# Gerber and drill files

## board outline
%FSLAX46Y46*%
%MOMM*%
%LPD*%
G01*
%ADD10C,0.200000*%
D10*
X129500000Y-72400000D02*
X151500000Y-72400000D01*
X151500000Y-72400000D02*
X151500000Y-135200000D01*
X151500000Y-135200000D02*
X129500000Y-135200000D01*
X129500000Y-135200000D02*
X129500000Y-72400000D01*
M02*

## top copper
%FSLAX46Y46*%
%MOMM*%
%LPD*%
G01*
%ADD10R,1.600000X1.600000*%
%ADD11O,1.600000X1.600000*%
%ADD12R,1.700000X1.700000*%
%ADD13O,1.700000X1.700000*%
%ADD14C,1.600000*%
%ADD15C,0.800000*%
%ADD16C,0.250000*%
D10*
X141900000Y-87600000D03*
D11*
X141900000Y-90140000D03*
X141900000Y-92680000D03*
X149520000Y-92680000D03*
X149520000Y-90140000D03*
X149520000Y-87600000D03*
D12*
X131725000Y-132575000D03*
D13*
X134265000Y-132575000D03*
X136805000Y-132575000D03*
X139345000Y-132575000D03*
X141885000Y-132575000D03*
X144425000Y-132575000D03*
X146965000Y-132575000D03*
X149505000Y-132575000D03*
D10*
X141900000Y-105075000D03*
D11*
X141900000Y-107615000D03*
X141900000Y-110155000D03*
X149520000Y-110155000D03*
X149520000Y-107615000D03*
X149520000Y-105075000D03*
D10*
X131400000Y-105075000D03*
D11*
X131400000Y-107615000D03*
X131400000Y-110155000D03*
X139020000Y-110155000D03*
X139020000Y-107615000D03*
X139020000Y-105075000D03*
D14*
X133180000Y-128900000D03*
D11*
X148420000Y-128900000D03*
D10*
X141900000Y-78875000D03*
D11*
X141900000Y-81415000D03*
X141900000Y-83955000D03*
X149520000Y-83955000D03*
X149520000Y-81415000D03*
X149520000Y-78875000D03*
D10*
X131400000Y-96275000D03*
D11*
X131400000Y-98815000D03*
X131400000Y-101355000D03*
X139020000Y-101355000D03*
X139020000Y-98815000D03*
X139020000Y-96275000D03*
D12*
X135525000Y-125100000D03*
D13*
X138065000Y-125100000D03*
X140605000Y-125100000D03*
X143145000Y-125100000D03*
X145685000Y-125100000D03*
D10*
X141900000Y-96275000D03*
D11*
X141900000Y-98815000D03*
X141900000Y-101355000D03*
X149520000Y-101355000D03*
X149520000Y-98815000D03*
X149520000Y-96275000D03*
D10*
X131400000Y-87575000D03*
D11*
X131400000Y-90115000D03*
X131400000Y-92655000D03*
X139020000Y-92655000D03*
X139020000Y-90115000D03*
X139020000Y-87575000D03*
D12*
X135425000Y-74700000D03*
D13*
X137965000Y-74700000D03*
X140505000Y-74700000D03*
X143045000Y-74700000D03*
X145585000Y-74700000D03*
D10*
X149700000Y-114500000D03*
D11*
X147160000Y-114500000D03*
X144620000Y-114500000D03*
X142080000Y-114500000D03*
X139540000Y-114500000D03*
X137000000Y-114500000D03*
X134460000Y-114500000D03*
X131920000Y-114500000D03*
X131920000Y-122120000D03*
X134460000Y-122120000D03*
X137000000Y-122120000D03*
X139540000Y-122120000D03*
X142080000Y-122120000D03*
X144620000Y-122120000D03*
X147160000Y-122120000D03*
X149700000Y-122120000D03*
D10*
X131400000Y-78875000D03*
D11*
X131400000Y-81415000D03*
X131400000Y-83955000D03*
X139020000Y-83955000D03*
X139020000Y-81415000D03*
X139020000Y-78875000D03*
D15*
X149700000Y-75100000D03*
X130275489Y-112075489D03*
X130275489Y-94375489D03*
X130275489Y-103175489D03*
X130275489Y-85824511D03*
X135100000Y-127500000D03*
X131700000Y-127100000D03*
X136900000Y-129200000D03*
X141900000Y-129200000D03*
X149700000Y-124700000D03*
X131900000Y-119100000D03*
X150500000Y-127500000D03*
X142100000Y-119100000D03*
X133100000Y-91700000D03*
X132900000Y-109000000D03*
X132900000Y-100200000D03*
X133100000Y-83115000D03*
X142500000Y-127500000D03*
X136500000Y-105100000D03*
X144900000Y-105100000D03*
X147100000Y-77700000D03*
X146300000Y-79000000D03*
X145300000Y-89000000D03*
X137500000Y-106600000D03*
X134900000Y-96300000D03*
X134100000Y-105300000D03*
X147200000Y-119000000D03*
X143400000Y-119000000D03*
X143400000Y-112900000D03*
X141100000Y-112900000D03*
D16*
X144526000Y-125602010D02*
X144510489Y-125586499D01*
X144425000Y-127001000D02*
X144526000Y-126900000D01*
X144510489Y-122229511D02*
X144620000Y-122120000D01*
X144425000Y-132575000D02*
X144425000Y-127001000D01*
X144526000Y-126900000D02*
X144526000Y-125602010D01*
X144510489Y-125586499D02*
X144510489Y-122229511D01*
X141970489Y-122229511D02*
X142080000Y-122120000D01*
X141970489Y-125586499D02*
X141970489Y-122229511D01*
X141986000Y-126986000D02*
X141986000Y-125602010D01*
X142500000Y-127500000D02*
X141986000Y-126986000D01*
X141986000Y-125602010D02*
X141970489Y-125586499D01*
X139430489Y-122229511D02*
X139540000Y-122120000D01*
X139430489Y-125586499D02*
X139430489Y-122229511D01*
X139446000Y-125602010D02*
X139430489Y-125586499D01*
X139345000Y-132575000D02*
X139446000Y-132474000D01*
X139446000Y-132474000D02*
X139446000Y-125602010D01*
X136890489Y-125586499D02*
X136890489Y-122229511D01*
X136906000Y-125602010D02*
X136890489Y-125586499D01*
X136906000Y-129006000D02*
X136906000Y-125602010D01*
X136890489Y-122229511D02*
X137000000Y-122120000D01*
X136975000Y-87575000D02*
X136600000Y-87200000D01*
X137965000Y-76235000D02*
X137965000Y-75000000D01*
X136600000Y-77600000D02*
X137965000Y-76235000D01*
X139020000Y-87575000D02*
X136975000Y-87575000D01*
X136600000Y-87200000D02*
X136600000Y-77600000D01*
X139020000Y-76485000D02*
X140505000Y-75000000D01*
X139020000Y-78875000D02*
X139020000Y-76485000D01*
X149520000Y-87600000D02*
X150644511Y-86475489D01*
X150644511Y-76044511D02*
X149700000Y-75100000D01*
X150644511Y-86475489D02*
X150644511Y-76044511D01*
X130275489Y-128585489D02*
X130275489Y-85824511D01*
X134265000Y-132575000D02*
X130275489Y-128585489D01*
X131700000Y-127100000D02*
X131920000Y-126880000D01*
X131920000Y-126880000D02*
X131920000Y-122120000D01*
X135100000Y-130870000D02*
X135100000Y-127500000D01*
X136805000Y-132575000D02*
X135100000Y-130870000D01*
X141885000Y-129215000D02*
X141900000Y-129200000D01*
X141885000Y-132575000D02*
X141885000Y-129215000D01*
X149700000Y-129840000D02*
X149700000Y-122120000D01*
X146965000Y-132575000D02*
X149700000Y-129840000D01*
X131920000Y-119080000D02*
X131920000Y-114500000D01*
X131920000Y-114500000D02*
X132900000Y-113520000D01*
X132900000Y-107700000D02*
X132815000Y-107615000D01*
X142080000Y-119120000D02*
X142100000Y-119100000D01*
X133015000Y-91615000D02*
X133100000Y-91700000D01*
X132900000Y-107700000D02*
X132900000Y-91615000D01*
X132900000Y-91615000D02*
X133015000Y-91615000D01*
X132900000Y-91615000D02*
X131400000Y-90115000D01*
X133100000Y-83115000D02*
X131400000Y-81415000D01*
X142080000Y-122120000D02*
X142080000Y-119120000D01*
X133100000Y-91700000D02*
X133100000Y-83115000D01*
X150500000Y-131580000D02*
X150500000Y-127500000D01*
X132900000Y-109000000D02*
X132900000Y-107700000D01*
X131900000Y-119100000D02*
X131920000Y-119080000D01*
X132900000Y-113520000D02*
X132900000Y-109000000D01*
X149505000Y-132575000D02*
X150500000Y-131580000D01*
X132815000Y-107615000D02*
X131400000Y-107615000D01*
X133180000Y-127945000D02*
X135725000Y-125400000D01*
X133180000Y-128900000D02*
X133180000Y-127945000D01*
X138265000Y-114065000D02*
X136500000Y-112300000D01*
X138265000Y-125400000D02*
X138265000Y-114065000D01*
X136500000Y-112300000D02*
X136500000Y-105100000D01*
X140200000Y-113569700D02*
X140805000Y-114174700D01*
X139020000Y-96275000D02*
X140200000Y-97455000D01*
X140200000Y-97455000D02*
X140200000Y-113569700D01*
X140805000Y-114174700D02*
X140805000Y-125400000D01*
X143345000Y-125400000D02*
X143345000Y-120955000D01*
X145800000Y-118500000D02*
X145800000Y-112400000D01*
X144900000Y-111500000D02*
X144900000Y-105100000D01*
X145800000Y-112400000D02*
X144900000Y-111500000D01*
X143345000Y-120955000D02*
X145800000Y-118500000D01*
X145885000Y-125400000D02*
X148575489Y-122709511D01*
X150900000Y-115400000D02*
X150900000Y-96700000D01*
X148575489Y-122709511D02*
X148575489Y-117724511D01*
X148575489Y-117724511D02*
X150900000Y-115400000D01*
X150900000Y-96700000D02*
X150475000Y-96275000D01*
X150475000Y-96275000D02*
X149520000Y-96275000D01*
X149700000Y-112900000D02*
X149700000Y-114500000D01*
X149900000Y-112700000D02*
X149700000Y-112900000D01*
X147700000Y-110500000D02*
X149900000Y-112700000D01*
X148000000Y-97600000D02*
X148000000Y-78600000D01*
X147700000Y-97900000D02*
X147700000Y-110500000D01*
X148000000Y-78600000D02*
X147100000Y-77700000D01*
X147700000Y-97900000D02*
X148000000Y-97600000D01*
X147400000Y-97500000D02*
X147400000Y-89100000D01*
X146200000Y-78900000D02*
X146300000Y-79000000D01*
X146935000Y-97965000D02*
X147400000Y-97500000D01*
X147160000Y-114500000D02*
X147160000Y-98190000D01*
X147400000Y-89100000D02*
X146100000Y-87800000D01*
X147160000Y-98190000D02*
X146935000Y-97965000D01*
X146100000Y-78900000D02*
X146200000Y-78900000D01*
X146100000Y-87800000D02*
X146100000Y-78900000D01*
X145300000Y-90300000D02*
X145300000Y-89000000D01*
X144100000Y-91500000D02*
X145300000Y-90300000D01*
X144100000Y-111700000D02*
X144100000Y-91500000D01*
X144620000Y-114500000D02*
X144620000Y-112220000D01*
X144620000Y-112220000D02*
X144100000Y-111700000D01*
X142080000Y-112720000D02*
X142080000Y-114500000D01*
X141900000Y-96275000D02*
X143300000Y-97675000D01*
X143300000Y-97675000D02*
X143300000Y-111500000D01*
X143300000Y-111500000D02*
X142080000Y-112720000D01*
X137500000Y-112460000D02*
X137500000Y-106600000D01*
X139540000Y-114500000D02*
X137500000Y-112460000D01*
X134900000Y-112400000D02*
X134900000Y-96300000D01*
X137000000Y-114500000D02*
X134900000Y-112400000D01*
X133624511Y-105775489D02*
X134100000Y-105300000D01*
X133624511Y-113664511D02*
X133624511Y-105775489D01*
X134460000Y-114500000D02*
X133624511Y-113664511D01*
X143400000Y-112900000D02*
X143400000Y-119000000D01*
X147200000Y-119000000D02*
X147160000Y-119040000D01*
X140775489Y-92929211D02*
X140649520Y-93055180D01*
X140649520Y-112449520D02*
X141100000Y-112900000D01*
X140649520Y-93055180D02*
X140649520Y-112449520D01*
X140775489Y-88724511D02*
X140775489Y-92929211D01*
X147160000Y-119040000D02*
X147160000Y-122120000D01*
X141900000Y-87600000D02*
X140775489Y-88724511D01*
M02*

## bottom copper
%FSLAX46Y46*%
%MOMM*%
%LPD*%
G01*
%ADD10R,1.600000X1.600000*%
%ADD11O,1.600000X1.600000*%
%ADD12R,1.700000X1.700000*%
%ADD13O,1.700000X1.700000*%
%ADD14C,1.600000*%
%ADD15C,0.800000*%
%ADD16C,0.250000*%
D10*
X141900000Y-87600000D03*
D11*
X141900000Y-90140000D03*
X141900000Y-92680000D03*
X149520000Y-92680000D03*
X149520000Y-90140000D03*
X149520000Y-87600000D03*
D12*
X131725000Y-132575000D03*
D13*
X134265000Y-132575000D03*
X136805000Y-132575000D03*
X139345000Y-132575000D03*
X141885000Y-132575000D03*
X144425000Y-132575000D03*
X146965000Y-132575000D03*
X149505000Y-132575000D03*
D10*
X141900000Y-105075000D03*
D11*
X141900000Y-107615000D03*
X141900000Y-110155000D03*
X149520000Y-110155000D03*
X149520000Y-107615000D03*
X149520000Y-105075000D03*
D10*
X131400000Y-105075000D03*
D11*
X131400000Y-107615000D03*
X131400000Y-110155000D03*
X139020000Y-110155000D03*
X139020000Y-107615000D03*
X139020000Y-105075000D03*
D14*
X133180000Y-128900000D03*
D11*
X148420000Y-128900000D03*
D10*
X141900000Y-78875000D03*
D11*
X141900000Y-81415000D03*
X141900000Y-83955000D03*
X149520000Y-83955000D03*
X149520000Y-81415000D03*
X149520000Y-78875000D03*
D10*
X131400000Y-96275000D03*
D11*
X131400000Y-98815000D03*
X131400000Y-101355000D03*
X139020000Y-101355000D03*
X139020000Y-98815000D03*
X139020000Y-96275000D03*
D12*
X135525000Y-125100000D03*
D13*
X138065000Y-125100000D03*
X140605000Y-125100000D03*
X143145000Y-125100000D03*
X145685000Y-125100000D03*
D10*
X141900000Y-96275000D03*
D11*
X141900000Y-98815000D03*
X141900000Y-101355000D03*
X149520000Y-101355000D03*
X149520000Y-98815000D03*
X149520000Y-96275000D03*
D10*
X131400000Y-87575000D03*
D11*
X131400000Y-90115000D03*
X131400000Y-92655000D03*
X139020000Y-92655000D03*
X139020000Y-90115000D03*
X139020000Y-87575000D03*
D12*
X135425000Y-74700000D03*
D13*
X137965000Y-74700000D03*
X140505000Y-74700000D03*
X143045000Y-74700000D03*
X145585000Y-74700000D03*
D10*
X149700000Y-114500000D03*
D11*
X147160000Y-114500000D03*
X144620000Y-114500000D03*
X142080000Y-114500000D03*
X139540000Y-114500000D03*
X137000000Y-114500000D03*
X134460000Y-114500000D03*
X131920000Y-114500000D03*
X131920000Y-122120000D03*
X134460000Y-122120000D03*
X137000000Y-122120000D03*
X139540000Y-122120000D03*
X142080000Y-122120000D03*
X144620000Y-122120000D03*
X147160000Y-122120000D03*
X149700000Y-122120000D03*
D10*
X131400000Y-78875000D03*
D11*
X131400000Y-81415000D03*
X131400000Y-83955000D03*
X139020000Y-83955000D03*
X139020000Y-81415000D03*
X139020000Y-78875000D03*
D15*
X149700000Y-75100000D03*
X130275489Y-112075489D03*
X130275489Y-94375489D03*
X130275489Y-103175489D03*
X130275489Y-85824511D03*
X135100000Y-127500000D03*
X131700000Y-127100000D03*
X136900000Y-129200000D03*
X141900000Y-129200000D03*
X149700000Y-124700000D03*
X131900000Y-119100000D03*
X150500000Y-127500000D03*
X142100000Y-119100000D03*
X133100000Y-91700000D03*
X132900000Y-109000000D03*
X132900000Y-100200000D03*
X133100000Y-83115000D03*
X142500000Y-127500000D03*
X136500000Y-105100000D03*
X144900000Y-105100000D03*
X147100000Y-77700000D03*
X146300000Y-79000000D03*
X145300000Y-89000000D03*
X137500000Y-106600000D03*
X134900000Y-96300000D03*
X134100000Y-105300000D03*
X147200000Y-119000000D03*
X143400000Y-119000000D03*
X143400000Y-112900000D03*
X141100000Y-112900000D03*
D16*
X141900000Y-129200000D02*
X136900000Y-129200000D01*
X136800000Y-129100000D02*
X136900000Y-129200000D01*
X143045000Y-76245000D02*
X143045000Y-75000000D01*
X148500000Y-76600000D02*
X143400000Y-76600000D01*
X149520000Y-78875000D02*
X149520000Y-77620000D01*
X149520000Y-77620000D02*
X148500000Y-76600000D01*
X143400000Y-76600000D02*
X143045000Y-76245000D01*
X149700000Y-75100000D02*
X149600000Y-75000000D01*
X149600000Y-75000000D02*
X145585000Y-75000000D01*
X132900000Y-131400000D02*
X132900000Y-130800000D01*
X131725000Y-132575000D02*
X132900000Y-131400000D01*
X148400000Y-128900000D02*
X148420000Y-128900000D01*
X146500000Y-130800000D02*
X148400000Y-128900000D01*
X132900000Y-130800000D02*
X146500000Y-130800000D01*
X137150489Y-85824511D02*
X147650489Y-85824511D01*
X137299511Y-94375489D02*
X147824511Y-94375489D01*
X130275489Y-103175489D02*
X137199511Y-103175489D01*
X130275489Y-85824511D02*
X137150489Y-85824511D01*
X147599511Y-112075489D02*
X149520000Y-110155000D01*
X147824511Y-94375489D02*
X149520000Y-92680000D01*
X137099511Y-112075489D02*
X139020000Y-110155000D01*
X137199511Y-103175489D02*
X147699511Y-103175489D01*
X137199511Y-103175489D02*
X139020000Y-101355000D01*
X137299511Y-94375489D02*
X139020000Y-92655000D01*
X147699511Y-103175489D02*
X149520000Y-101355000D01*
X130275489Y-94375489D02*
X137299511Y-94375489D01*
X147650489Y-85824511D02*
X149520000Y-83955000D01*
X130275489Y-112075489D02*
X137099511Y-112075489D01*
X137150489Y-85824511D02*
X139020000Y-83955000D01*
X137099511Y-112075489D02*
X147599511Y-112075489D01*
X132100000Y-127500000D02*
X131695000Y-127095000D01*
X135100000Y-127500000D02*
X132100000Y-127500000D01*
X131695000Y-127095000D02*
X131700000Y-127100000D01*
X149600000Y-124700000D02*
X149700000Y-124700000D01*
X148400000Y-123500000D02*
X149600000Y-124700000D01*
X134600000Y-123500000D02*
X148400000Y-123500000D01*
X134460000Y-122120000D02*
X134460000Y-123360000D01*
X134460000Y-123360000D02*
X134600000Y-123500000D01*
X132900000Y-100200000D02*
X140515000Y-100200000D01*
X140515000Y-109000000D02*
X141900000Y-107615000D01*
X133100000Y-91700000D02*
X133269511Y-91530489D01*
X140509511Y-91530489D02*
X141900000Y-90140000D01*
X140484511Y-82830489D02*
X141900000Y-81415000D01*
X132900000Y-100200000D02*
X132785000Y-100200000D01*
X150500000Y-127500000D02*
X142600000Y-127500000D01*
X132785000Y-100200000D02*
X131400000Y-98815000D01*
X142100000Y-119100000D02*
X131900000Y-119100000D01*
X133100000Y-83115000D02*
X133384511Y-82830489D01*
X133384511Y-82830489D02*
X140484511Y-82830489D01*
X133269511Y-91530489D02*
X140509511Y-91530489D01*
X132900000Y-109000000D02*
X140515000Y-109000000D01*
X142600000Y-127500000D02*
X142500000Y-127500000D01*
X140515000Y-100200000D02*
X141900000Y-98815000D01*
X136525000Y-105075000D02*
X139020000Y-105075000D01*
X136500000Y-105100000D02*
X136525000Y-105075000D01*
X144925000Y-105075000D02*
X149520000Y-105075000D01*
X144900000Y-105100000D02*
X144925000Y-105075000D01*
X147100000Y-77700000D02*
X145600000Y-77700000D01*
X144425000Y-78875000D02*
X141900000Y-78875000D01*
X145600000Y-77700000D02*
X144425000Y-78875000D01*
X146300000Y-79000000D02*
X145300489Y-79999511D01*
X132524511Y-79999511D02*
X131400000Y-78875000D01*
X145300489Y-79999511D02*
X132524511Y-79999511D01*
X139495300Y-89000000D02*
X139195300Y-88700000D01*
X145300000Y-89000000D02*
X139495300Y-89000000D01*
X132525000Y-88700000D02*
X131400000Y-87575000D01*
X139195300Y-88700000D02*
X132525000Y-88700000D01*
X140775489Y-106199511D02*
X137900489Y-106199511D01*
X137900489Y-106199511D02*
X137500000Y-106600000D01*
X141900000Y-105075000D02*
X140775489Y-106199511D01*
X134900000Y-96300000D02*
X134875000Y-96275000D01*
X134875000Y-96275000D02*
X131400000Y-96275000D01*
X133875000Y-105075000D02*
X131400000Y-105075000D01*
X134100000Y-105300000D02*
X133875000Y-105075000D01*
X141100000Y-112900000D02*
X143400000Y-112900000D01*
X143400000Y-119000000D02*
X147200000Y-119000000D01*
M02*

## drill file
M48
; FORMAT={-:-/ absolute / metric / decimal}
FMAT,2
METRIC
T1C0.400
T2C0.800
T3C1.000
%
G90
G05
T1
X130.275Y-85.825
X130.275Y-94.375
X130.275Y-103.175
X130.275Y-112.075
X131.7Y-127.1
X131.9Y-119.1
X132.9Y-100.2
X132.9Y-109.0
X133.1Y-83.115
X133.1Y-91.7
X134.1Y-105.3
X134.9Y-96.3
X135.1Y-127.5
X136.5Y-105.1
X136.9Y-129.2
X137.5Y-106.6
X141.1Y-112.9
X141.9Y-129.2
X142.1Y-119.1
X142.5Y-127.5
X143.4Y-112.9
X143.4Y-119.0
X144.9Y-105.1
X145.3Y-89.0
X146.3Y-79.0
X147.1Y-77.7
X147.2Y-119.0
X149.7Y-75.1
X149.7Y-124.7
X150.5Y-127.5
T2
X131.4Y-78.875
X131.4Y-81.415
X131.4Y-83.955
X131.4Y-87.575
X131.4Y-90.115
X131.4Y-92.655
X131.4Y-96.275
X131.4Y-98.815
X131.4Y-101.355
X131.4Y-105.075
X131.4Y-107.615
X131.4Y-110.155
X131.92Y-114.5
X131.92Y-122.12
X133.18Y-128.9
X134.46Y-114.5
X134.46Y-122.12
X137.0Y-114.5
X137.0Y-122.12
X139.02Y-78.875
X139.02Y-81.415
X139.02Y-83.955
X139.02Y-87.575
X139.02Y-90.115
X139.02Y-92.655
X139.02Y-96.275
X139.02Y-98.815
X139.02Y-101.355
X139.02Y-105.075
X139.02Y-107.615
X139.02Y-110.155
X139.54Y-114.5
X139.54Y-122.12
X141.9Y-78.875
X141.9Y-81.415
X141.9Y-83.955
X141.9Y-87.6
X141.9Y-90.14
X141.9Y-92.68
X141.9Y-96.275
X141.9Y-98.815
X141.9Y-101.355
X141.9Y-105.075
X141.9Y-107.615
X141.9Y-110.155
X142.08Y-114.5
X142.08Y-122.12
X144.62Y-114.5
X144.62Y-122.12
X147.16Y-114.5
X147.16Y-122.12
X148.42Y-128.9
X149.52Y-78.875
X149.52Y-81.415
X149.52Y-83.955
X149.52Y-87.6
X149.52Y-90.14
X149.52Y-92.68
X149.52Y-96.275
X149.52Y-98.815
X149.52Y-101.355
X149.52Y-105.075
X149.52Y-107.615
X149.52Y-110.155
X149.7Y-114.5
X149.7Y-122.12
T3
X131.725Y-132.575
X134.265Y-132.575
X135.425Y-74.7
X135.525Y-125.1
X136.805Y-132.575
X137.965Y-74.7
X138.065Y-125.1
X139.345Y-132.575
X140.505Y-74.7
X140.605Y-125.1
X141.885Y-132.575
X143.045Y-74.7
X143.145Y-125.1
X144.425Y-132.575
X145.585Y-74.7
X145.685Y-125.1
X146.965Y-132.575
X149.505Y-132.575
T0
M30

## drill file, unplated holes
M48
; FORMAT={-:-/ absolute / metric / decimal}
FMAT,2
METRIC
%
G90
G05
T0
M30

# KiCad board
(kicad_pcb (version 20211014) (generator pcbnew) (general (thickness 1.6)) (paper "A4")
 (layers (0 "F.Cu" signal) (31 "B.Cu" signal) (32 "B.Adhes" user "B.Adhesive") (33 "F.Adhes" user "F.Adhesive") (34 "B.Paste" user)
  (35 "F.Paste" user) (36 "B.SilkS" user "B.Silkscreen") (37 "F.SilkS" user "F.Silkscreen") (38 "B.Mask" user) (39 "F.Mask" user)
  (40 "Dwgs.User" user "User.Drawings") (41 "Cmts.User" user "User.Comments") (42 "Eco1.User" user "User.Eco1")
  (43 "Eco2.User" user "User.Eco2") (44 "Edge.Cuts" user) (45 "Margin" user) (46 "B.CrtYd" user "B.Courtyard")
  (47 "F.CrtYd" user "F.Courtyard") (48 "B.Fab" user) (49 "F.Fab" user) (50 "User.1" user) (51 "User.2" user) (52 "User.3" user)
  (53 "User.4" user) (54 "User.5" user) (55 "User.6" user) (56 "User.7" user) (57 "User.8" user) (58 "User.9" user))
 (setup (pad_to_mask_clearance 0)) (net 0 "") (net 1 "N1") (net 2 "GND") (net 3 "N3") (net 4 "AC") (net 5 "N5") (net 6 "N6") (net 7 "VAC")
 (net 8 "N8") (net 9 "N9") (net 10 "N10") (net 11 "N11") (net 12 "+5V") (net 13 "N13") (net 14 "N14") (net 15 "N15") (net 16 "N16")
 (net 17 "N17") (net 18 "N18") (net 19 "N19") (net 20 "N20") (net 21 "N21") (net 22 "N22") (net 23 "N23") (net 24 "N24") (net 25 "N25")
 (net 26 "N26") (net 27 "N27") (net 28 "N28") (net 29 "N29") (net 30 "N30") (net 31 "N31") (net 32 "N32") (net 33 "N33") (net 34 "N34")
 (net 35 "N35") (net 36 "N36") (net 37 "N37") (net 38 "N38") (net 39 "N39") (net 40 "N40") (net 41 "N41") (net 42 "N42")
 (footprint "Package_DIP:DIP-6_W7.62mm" (layer "F.Cu") (at 141.9 87.6)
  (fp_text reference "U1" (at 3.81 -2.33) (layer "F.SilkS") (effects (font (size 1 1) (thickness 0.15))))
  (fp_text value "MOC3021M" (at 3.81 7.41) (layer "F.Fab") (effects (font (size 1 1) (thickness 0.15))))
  (pad "1" thru_hole rect (at 0 0) (size 1.6 1.6) (drill 0.8) (layers *.Cu *.Mask) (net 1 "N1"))
  (pad "2" thru_hole oval (at 0 2.54) (size 1.6 1.6) (drill 0.8) (layers *.Cu *.Mask) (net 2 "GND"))
  (pad "3" thru_hole oval (at 0 5.08) (size 1.6 1.6) (drill 0.8) (layers *.Cu *.Mask) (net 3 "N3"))
  (pad "4" thru_hole oval (at 7.62 5.08) (size 1.6 1.6) (drill 0.8) (layers *.Cu *.Mask) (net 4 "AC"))
  (pad "5" thru_hole oval (at 7.62 2.54) (size 1.6 1.6) (drill 0.8) (layers *.Cu *.Mask) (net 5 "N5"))
  (pad "6" thru_hole oval (at 7.62 0) (size 1.6 1.6) (drill 0.8) (layers *.Cu *.Mask) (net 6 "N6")))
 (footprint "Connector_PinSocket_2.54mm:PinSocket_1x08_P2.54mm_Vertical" (layer "F.Cu") (at 131.725 132.575 90)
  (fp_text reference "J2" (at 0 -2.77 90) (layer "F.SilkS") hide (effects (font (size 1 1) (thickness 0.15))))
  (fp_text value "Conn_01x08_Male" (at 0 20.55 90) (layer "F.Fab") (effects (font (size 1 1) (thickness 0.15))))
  (pad "1" thru_hole rect (at 0 0 90) (size 1.7 1.7) (drill 1) (layers *.Cu *.Mask) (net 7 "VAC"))
  (pad "2" thru_hole oval (at 0 2.54 90) (size 1.7 1.7) (drill 1) (layers *.Cu *.Mask) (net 4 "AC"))
  (pad "3" thru_hole oval (at 0 5.08 90) (size 1.7 1.7) (drill 1) (layers *.Cu *.Mask) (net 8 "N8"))
  (pad "4" thru_hole oval (at 0 7.62 90) (size 1.7 1.7) (drill 1) (layers *.Cu *.Mask) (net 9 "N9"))
  (pad "5" thru_hole oval (at 0 10.16 90) (size 1.7 1.7) (drill 1) (layers *.Cu *.Mask) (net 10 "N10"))
  (pad "6" thru_hole oval (at 0 12.7 90) (size 1.7 1.7) (drill 1) (layers *.Cu *.Mask) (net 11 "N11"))
  (pad "7" thru_hole oval (at 0 15.24 90) (size 1.7 1.7) (drill 1) (layers *.Cu *.Mask) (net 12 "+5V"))
  (pad "8" thru_hole oval (at 0 17.78 90) (size 1.7 1.7) (drill 1) (layers *.Cu *.Mask) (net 2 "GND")))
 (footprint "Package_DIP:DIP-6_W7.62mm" (layer "F.Cu") (at 141.9 105.075)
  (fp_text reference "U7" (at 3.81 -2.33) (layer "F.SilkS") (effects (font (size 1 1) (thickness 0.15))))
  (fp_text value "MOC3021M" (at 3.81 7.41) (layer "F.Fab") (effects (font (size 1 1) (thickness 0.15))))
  (pad "1" thru_hole rect (at 0 0) (size 1.6 1.6) (drill 0.8) (layers *.Cu *.Mask) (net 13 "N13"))
  (pad "2" thru_hole oval (at 0 2.54) (size 1.6 1.6) (drill 0.8) (layers *.Cu *.Mask) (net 2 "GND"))
  (pad "3" thru_hole oval (at 0 5.08) (size 1.6 1.6) (drill 0.8) (layers *.Cu *.Mask) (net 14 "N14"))
  (pad "4" thru_hole oval (at 7.62 5.08) (size 1.6 1.6) (drill 0.8) (layers *.Cu *.Mask) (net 4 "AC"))
  (pad "5" thru_hole oval (at 7.62 2.54) (size 1.6 1.6) (drill 0.8) (layers *.Cu *.Mask) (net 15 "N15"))
  (pad "6" thru_hole oval (at 7.62 0) (size 1.6 1.6) (drill 0.8) (layers *.Cu *.Mask) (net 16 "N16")))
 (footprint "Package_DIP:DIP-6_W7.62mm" (layer "F.Cu") (at 131.4 105.075)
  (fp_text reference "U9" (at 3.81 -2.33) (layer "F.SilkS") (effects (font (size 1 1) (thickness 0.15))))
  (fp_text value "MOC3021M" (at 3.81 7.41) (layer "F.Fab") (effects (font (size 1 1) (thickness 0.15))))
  (pad "1" thru_hole rect (at 0 0) (size 1.6 1.6) (drill 0.8) (layers *.Cu *.Mask) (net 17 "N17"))
  (pad "2" thru_hole oval (at 0 2.54) (size 1.6 1.6) (drill 0.8) (layers *.Cu *.Mask) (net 2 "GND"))
  (pad "3" thru_hole oval (at 0 5.08) (size 1.6 1.6) (drill 0.8) (layers *.Cu *.Mask) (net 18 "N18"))
  (pad "4" thru_hole oval (at 7.62 5.08) (size 1.6 1.6) (drill 0.8) (layers *.Cu *.Mask) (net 4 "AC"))
  (pad "5" thru_hole oval (at 7.62 2.54) (size 1.6 1.6) (drill 0.8) (layers *.Cu *.Mask) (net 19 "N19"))
  (pad "6" thru_hole oval (at 7.62 0) (size 1.6 1.6) (drill 0.8) (layers *.Cu *.Mask) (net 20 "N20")))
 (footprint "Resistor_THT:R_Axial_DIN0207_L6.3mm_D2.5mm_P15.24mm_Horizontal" (layer "F.Cu") (at 133.18 128.9)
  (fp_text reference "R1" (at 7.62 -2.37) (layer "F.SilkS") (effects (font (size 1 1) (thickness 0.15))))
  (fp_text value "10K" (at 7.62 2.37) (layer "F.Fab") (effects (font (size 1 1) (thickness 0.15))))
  (pad "1" thru_hole circle (at 0 0) (size 1.6 1.6) (drill 0.8) (layers *.Cu *.Mask) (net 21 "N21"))
  (pad "2" thru_hole oval (at 15.24 0) (size 1.6 1.6) (drill 0.8) (layers *.Cu *.Mask) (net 7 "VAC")))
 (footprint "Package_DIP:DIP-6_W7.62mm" (layer "F.Cu") (at 141.9 78.875)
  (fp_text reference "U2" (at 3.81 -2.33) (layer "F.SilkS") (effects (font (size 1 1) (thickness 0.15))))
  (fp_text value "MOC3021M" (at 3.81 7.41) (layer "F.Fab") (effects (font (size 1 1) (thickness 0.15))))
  (pad "1" thru_hole rect (at 0 0) (size 1.6 1.6) (drill 0.8) (layers *.Cu *.Mask) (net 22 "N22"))
  (pad "2" thru_hole oval (at 0 2.54) (size 1.6 1.6) (drill 0.8) (layers *.Cu *.Mask) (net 2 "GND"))
  (pad "3" thru_hole oval (at 0 5.08) (size 1.6 1.6) (drill 0.8) (layers *.Cu *.Mask) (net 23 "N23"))
  (pad "4" thru_hole oval (at 7.62 5.08) (size 1.6 1.6) (drill 0.8) (layers *.Cu *.Mask) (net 4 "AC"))
  (pad "5" thru_hole oval (at 7.62 2.54) (size 1.6 1.6) (drill 0.8) (layers *.Cu *.Mask) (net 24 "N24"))
  (pad "6" thru_hole oval (at 7.62 0) (size 1.6 1.6) (drill 0.8) (layers *.Cu *.Mask) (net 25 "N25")))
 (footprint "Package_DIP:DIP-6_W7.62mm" (layer "F.Cu") (at 131.4 96.275)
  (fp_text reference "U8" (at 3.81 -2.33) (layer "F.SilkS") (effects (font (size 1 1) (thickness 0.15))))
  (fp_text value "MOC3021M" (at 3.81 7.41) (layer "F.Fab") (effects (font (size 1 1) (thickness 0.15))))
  (pad "1" thru_hole rect (at 0 0) (size 1.6 1.6) (drill 0.8) (layers *.Cu *.Mask) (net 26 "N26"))
  (pad "2" thru_hole oval (at 0 2.54) (size 1.6 1.6) (drill 0.8) (layers *.Cu *.Mask) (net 2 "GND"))
  (pad "3" thru_hole oval (at 0 5.08) (size 1.6 1.6) (drill 0.8) (layers *.Cu *.Mask) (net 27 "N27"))
  (pad "4" thru_hole oval (at 7.62 5.08) (size 1.6 1.6) (drill 0.8) (layers *.Cu *.Mask) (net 4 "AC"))
  (pad "5" thru_hole oval (at 7.62 2.54) (size 1.6 1.6) (drill 0.8) (layers *.Cu *.Mask) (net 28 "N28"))
  (pad "6" thru_hole oval (at 7.62 0) (size 1.6 1.6) (drill 0.8) (layers *.Cu *.Mask) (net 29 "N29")))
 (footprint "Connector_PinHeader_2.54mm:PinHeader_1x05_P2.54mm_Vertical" (layer "F.Cu") (at 135.525 125.1 90)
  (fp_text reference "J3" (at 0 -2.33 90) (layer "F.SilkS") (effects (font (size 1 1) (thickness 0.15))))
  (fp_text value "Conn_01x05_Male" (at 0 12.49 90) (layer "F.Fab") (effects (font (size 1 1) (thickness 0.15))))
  (pad "1" thru_hole rect (at 0 0 90) (size 1.7 1.7) (drill 1) (layers *.Cu *.Mask) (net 21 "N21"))
  (pad "2" thru_hole oval (at 0 2.54 90) (size 1.7 1.7) (drill 1) (layers *.Cu *.Mask) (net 20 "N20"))
  (pad "3" thru_hole oval (at 0 5.08 90) (size 1.7 1.7) (drill 1) (layers *.Cu *.Mask) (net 29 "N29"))
  (pad "4" thru_hole oval (at 0 7.62 90) (size 1.7 1.7) (drill 1) (layers *.Cu *.Mask) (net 16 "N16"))
  (pad "5" thru_hole oval (at 0 10.16 90) (size 1.7 1.7) (drill 1) (layers *.Cu *.Mask) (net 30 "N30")))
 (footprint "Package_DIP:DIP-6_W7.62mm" (layer "F.Cu") (at 141.9 96.275)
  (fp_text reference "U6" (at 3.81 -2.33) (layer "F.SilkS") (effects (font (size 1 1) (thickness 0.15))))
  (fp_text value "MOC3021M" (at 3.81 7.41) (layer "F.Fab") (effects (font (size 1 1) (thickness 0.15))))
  (pad "1" thru_hole rect (at 0 0) (size 1.6 1.6) (drill 0.8) (layers *.Cu *.Mask) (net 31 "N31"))
  (pad "2" thru_hole oval (at 0 2.54) (size 1.6 1.6) (drill 0.8) (layers *.Cu *.Mask) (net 2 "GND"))
  (pad "3" thru_hole oval (at 0 5.08) (size 1.6 1.6) (drill 0.8) (layers *.Cu *.Mask) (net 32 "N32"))
  (pad "4" thru_hole oval (at 7.62 5.08) (size 1.6 1.6) (drill 0.8) (layers *.Cu *.Mask) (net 4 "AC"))
  (pad "5" thru_hole oval (at 7.62 2.54) (size 1.6 1.6) (drill 0.8) (layers *.Cu *.Mask) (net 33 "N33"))
  (pad "6" thru_hole oval (at 7.62 0) (size 1.6 1.6) (drill 0.8) (layers *.Cu *.Mask) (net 30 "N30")))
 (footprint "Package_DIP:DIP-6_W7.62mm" (layer "F.Cu") (at 131.4 87.575)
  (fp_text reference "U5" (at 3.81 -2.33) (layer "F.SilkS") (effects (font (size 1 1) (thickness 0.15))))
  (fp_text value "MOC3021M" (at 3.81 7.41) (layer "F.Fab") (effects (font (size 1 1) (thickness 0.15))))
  (pad "1" thru_hole rect (at 0 0) (size 1.6 1.6) (drill 0.8) (layers *.Cu *.Mask) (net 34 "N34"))
  (pad "2" thru_hole oval (at 0 2.54) (size 1.6 1.6) (drill 0.8) (layers *.Cu *.Mask) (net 2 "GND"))
  (pad "3" thru_hole oval (at 0 5.08) (size 1.6 1.6) (drill 0.8) (layers *.Cu *.Mask) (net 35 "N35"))
  (pad "4" thru_hole oval (at 7.62 5.08) (size 1.6 1.6) (drill 0.8) (layers *.Cu *.Mask) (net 4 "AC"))
  (pad "5" thru_hole oval (at 7.62 2.54) (size 1.6 1.6) (drill 0.8) (layers *.Cu *.Mask) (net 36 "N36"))
  (pad "6" thru_hole oval (at 7.62 0) (size 1.6 1.6) (drill 0.8) (layers *.Cu *.Mask) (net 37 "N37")))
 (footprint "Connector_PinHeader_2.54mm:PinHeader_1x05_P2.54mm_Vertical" (layer "F.Cu") (at 135.425 74.7 90)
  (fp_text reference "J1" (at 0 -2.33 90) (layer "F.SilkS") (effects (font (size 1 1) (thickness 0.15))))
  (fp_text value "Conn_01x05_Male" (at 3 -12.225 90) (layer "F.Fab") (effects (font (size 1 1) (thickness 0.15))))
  (pad "1" thru_hole rect (at 0 0 90) (size 1.7 1.7) (drill 1) (layers *.Cu *.Mask) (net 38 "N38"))
  (pad "2" thru_hole oval (at 0 2.54 90) (size 1.7 1.7) (drill 1) (layers *.Cu *.Mask) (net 37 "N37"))
  (pad "3" thru_hole oval (at 0 5.08 90) (size 1.7 1.7) (drill 1) (layers *.Cu *.Mask) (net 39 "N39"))
  (pad "4" thru_hole oval (at 0 7.62 90) (size 1.7 1.7) (drill 1) (layers *.Cu *.Mask) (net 25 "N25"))
  (pad "5" thru_hole oval (at 0 10.16 90) (size 1.7 1.7) (drill 1) (layers *.Cu *.Mask) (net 6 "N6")))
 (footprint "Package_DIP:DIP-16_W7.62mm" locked (layer "F.Cu") (at 149.7 114.5 -90)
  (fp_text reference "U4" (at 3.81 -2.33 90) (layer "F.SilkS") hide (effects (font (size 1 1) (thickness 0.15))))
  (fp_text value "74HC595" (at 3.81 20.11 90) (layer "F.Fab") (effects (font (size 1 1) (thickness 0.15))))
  (pad "1" thru_hole rect locked (at 0 0 270) (size 1.6 1.6) (drill 0.8) (layers *.Cu *.Mask) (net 22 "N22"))
  (pad "2" thru_hole oval locked (at 0 2.54 270) (size 1.6 1.6) (drill 0.8) (layers *.Cu *.Mask) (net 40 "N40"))
  (pad "3" thru_hole oval locked (at 0 5.08 270) (size 1.6 1.6) (drill 0.8) (layers *.Cu *.Mask) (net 34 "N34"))
  (pad "4" thru_hole oval locked (at 0 7.62 270) (size 1.6 1.6) (drill 0.8) (layers *.Cu *.Mask) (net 31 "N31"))
  (pad "5" thru_hole oval locked (at 0 10.16 270) (size 1.6 1.6) (drill 0.8) (layers *.Cu *.Mask) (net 13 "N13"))
  (pad "6" thru_hole oval locked (at 0 12.7 270) (size 1.6 1.6) (drill 0.8) (layers *.Cu *.Mask) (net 26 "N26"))
  (pad "7" thru_hole oval locked (at 0 15.24 270) (size 1.6 1.6) (drill 0.8) (layers *.Cu *.Mask) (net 17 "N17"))
  (pad "8" thru_hole oval locked (at 0 17.78 270) (size 1.6 1.6) (drill 0.8) (layers *.Cu *.Mask) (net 2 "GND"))
  (pad "9" thru_hole oval locked (at 7.62 17.78 270) (size 1.6 1.6) (drill 0.8) (layers *.Cu *.Mask) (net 8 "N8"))
  (pad "10" thru_hole oval locked (at 7.62 15.24 270) (size 1.6 1.6) (drill 0.8) (layers *.Cu *.Mask) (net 12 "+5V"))
  (pad "11" thru_hole oval locked (at 7.62 12.7 270) (size 1.6 1.6) (drill 0.8) (layers *.Cu *.Mask) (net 10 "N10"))
  (pad "12" thru_hole oval locked (at 7.62 10.16 270) (size 1.6 1.6) (drill 0.8) (layers *.Cu *.Mask) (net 9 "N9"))
  (pad "13" thru_hole oval locked (at 7.62 7.62 270) (size 1.6 1.6) (drill 0.8) (layers *.Cu *.Mask) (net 2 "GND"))
  (pad "14" thru_hole oval locked (at 7.62 5.08 270) (size 1.6 1.6) (drill 0.8) (layers *.Cu *.Mask) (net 11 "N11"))
  (pad "15" thru_hole oval locked (at 7.62 2.54 270) (size 1.6 1.6) (drill 0.8) (layers *.Cu *.Mask) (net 1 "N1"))
  (pad "16" thru_hole oval locked (at 7.62 0 270) (size 1.6 1.6) (drill 0.8) (layers *.Cu *.Mask) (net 12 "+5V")))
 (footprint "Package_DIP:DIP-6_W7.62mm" (layer "F.Cu") (at 131.4 78.875)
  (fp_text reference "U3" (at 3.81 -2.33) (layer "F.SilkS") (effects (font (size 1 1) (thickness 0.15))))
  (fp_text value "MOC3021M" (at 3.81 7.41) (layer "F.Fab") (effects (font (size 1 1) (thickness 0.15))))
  (pad "1" thru_hole rect (at 0 0) (size 1.6 1.6) (drill 0.8) (layers *.Cu *.Mask) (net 40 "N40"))
  (pad "2" thru_hole oval (at 0 2.54) (size 1.6 1.6) (drill 0.8) (layers *.Cu *.Mask) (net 2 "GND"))
  (pad "3" thru_hole oval (at 0 5.08) (size 1.6 1.6) (drill 0.8) (layers *.Cu *.Mask) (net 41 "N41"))
  (pad "4" thru_hole oval (at 7.62 5.08) (size 1.6 1.6) (drill 0.8) (layers *.Cu *.Mask) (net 4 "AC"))
  (pad "5" thru_hole oval (at 7.62 2.54) (size 1.6 1.6) (drill 0.8) (layers *.Cu *.Mask) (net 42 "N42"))
  (pad "6" thru_hole oval (at 7.62 0) (size 1.6 1.6) (drill 0.8) (layers *.Cu *.Mask) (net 39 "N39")))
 (gr_rect (start 129.5 72.4) (end 151.5 135.2) (layer "Edge.Cuts") (width 0.2) (fill none))
 (segment (start 136.975 87.575) (end 136.6 87.2) (width 0.25) (layer "F.Cu") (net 37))
 (segment (start 137.965 76.235) (end 137.965 75) (width 0.25) (layer "F.Cu") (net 37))
 (segment (start 136.6 77.6) (end 137.965 76.235) (width 0.25) (layer "F.Cu") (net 37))
 (segment (start 139.02 87.575) (end 136.975 87.575) (width 0.25) (layer "F.Cu") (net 37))
 (segment (start 136.6 87.2) (end 136.6 77.6) (width 0.25) (layer "F.Cu") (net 37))
 (segment (start 139.02 76.485) (end 140.505 75) (width 0.25) (layer "F.Cu") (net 39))
 (segment (start 139.02 78.875) (end 139.02 76.485) (width 0.25) (layer "F.Cu") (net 39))
 (segment (start 143.045 76.245) (end 143.045 75) (width 0.25) (layer "B.Cu") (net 25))
 (segment (start 148.5 76.6) (end 143.4 76.6) (width 0.25) (layer "B.Cu") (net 25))
 (segment (start 149.52 78.875) (end 149.52 77.62) (width 0.25) (layer "B.Cu") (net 25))
 (segment (start 149.52 77.62) (end 148.5 76.6) (width 0.25) (layer "B.Cu") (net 25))
 (segment (start 143.4 76.6) (end 143.045 76.245) (width 0.25) (layer "B.Cu") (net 25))
 (segment (start 149.52 87.6) (end 150.644511 86.475489) (width 0.25) (layer "F.Cu") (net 6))
 (segment (start 150.644511 76.044511) (end 149.7 75.1) (width 0.25) (layer "F.Cu") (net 6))
 (segment (start 150.644511 86.475489) (end 150.644511 76.044511) (width 0.25) (layer "F.Cu") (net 6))
 (via (at 149.7 75.1) (size 0.8) (drill 0.4) (layers "F.Cu" "B.Cu") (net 6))
 (segment (start 149.7 75.1) (end 149.6 75) (width 0.25) (layer "B.Cu") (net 6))
 (segment (start 149.6 75) (end 145.585 75) (width 0.25) (layer "B.Cu") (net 6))
 (segment (start 132.9 131.4) (end 132.9 130.8) (width 0.25) (layer "B.Cu") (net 7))
 (segment (start 131.725 132.575) (end 132.9 131.4) (width 0.25) (layer "B.Cu") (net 7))
 (segment (start 148.4 128.9) (end 148.42 128.9) (width 0.25) (layer "B.Cu") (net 7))
 (segment (start 146.5 130.8) (end 148.4 128.9) (width 0.25) (layer "B.Cu") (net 7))
 (segment (start 132.9 130.8) (end 146.5 130.8) (width 0.25) (layer "B.Cu") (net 7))
 (segment (start 130.275489 128.585489) (end 130.275489 85.824511) (width 0.25) (layer "F.Cu") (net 4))
 (segment (start 134.265 132.575) (end 130.275489 128.585489) (width 0.25) (layer "F.Cu") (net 4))
 (via (at 130.275489 112.075489) (size 0.8) (drill 0.4) (layers "F.Cu" "B.Cu") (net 4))
 (via (at 130.275489 94.375489) (size 0.8) (drill 0.4) (layers "F.Cu" "B.Cu") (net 4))
 (via (at 130.275489 103.175489) (size 0.8) (drill 0.4) (layers "F.Cu" "B.Cu") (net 4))
 (via (at 130.275489 85.824511) (size 0.8) (drill 0.4) (layers "F.Cu" "B.Cu") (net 4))
 (segment (start 137.150489 85.824511) (end 147.650489 85.824511) (width 0.25) (layer "B.Cu") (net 4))
 (segment (start 137.299511 94.375489) (end 147.824511 94.375489) (width 0.25) (layer "B.Cu") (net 4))
 (segment (start 130.275489 103.175489) (end 137.199511 103.175489) (width 0.25) (layer "B.Cu") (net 4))
 (segment (start 130.275489 85.824511) (end 137.150489 85.824511) (width 0.25) (layer "B.Cu") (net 4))
 (segment (start 147.599511 112.075489) (end 149.52 110.155) (width 0.25) (layer "B.Cu") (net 4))
 (segment (start 147.824511 94.375489) (end 149.52 92.68) (width 0.25) (layer "B.Cu") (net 4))
 (segment (start 137.099511 112.075489) (end 139.02 110.155) (width 0.25) (layer "B.Cu") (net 4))
 (segment (start 137.199511 103.175489) (end 147.699511 103.175489) (width 0.25) (layer "B.Cu") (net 4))
 (segment (start 137.199511 103.175489) (end 139.02 101.355) (width 0.25) (layer "B.Cu") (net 4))
 (segment (start 137.299511 94.375489) (end 139.02 92.655) (width 0.25) (layer "B.Cu") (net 4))
 (segment (start 147.699511 103.175489) (end 149.52 101.355) (width 0.25) (layer "B.Cu") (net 4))
 (segment (start 130.275489 94.375489) (end 137.299511 94.375489) (width 0.25) (layer "B.Cu") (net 4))
 (segment (start 147.650489 85.824511) (end 149.52 83.955) (width 0.25) (layer "B.Cu") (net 4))
 (segment (start 130.275489 112.075489) (end 137.099511 112.075489) (width 0.25) (layer "B.Cu") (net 4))
 (segment (start 137.150489 85.824511) (end 139.02 83.955) (width 0.25) (layer "B.Cu") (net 4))
 (segment (start 137.099511 112.075489) (end 147.599511 112.075489) (width 0.25) (layer "B.Cu") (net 4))
 (segment (start 131.7 127.1) (end 131.92 126.88) (width 0.25) (layer "F.Cu") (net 8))
 (segment (start 131.92 126.88) (end 131.92 122.12) (width 0.25) (layer "F.Cu") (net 8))
 (segment (start 135.1 130.87) (end 135.1 127.5) (width 0.25) (layer "F.Cu") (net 8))
 (segment (start 136.805 132.575) (end 135.1 130.87) (width 0.25) (layer "F.Cu") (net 8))
 (via (at 135.1 127.5) (size 0.8) (drill 0.4) (layers "F.Cu" "B.Cu") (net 8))
 (via (at 131.7 127.1) (size 0.8) (drill 0.4) (layers "F.Cu" "B.Cu") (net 8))
 (segment (start 132.1 127.5) (end 131.695 127.095) (width 0.25) (layer "B.Cu") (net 8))
 (segment (start 135.1 127.5) (end 132.1 127.5) (width 0.25) (layer "B.Cu") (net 8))
 (segment (start 131.695 127.095) (end 131.7 127.1) (width 0.25) (layer "B.Cu") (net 8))
 (segment (start 139.430489 125.586499) (end 139.430489 122.229511) (width 0.25) (layer "F.Cu") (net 9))
 (segment (start 139.446 125.60201) (end 139.430489 125.586499) (width 0.25) (layer "F.Cu") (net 9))
 (segment (start 139.446 132.474) (end 139.446 125.60201) (width 0.25) (layer "F.Cu") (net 9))
 (segment (start 139.345 132.575) (end 139.446 132.474) (width 0.25) (layer "F.Cu") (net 9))
 (segment (start 139.430489 122.229511) (end 139.54 122.12) (width 0.25) (layer "F.Cu") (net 9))
 (segment (start 136.890489 122.229511) (end 137 122.12) (width 0.25) (layer "F.Cu") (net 10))
 (segment (start 141.885 129.215) (end 141.9 129.2) (width 0.25) (layer "F.Cu") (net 10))
 (segment (start 141.885 132.575) (end 141.885 129.215) (width 0.25) (layer "F.Cu") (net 10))
 (segment (start 136.890489 125.586499) (end 136.890489 122.229511) (width 0.25) (layer "F.Cu") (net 10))
 (segment (start 136.906 129.006) (end 136.906 125.60201) (width 0.25) (layer "F.Cu") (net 10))
 (segment (start 136.906 125.60201) (end 136.890489 125.586499) (width 0.25) (layer "F.Cu") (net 10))
 (via (at 136.9 129.2) (size 0.8) (drill 0.4) (layers "F.Cu" "B.Cu") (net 10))
 (via (at 141.9 129.2) (size 0.8) (drill 0.4) (layers "F.Cu" "B.Cu") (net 10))
 (segment (start 136.8 129.1) (end 136.9 129.2) (width 0.25) (layer "B.Cu") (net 10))
 (segment (start 141.9 129.2) (end 136.9 129.2) (width 0.25) (layer "B.Cu") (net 10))
 (segment (start 144.425 127.001) (end 144.526 126.9) (width 0.25) (layer "F.Cu") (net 11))
 (segment (start 144.526 125.60201) (end 144.510489 125.586499) (width 0.25) (layer "F.Cu") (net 11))
 (segment (start 144.425 132.575) (end 144.425 127.001) (width 0.25) (layer "F.Cu") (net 11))
 (segment (start 144.526 126.9) (end 144.526 125.60201) (width 0.25) (layer "F.Cu") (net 11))
 (segment (start 144.510489 125.586499) (end 144.510489 122.229511) (width 0.25) (layer "F.Cu") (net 11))
 (segment (start 144.510489 122.229511) (end 144.62 122.12) (width 0.25) (layer "F.Cu") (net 11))
 (segment locked (start 149.7 129.84) (end 149.7 122.12) (width 0.25) (layer "F.Cu") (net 12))
 (segment (start 146.965 132.575) (end 149.7 129.84) (width 0.25) (layer "F.Cu") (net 12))
 (via (at 149.7 124.7) (size 0.8) (drill 0.4) (layers "F.Cu" "B.Cu") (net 12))
 (segment (start 149.6 124.7) (end 149.7 124.7) (width 0.25) (layer "B.Cu") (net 12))
 (segment (start 148.4 123.5) (end 149.6 124.7) (width 0.25) (layer "B.Cu") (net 12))
 (segment (start 134.6 123.5) (end 148.4 123.5) (width 0.25) (layer "B.Cu") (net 12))
 (segment (start 134.46 122.12) (end 134.46 123.36) (width 0.25) (layer "B.Cu") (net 12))
 (segment (start 134.46 123.36) (end 134.6 123.5) (width 0.25) (layer "B.Cu") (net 12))
 (segment (start 131.92 119.08) (end 131.92 114.5) (width 0.25) (layer "F.Cu") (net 2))
 (segment (start 141.970489 122.229511) (end 142.08 122.12) (width 0.25) (layer "F.Cu") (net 2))
 (segment (start 131.92 114.5) (end 132.9 113.52) (width 0.25) (layer "F.Cu") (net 2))
 (segment (start 141.986 126.986) (end 141.986 125.60201) (width 0.25) (layer "F.Cu") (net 2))
 (segment (start 132.9 107.7) (end 132.815 107.615) (width 0.25) (layer "F.Cu") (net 2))
 (segment (start 142.08 119.12) (end 142.1 119.1) (width 0.25) (layer "F.Cu") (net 2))
 (segment (start 142.5 127.5) (end 141.986 126.986) (width 0.25) (layer "F.Cu") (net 2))
 (segment (start 133.015 91.615) (end 133.1 91.7) (width 0.25) (layer "F.Cu") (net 2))
 (segment (start 132.9 107.7) (end 132.9 91.615) (width 0.25) (layer "F.Cu") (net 2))
 (segment (start 132.9 91.615) (end 133.015 91.615) (width 0.25) (layer "F.Cu") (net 2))
 (segment (start 132.9 91.615) (end 131.4 90.115) (width 0.25) (layer "F.Cu") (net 2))
 (segment (start 133.1 83.115) (end 131.4 81.415) (width 0.25) (layer "F.Cu") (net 2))
 (segment (start 142.08 122.12) (end 142.08 119.12) (width 0.25) (layer "F.Cu") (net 2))
 (segment (start 133.1 91.7) (end 133.1 83.115) (width 0.25) (layer "F.Cu") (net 2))
 (segment (start 150.5 131.58) (end 150.5 127.5) (width 0.25) (layer "F.Cu") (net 2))
 (segment (start 132.9 109) (end 132.9 107.7) (width 0.25) (layer "F.Cu") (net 2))
 (segment (start 131.9 119.1) (end 131.92 119.08) (width 0.25) (layer "F.Cu") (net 2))
 (segment (start 141.970489 125.586499) (end 141.970489 122.229511) (width 0.25) (layer "F.Cu") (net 2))
 (segment (start 141.986 125.60201) (end 141.970489 125.586499) (width 0.25) (layer "F.Cu") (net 2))
 (segment (start 132.9 113.52) (end 132.9 109) (width 0.25) (layer "F.Cu") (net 2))
 (segment (start 149.505 132.575) (end 150.5 131.58) (width 0.25) (layer "F.Cu") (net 2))
 (segment (start 132.815 107.615) (end 131.4 107.615) (width 0.25) (layer "F.Cu") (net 2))
 (via (at 131.9 119.1) (size 0.8) (drill 0.4) (layers "F.Cu" "B.Cu") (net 2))
 (via (at 150.5 127.5) (size 0.8) (drill 0.4) (layers "F.Cu" "B.Cu") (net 2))
 (via (at 142.1 119.1) (size 0.8) (drill 0.4) (layers "F.Cu" "B.Cu") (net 2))
 (via (at 133.1 91.7) (size 0.8) (drill 0.4) (layers "F.Cu" "B.Cu") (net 2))
 (via (at 132.9 109) (size 0.8) (drill 0.4) (layers "F.Cu" "B.Cu") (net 2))
 (via (at 132.9 100.2) (size 0.8) (drill 0.4) (layers "F.Cu" "B.Cu") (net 2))
 (via (at 133.1 83.115) (size 0.8) (drill 0.4) (layers "F.Cu" "B.Cu") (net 2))
 (via (at 142.5 127.5) (size 0.8) (drill 0.4) (layers "F.Cu" "B.Cu") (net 2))
 (segment (start 132.9 100.2) (end 140.515 100.2) (width 0.25) (layer "B.Cu") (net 2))
 (segment (start 140.515 109) (end 141.9 107.615) (width 0.25) (layer "B.Cu") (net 2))
 (segment (start 133.1 91.7) (end 133.269511 91.530489) (width 0.25) (layer "B.Cu") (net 2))
 (segment (start 140.509511 91.530489) (end 141.9 90.14) (width 0.25) (layer "B.Cu") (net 2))
 (segment (start 140.484511 82.830489) (end 141.9 81.415) (width 0.25) (layer "B.Cu") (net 2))
 (segment (start 132.9 100.2) (end 132.785 100.2) (width 0.25) (layer "B.Cu") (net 2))
 (segment (start 150.5 127.5) (end 142.6 127.5) (width 0.25) (layer "B.Cu") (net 2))
 (segment (start 132.785 100.2) (end 131.4 98.815) (width 0.25) (layer "B.Cu") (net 2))
 (segment (start 142.1 119.1) (end 131.9 119.1) (width 0.25) (layer "B.Cu") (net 2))
 (segment (start 133.1 83.115) (end 133.384511 82.830489) (width 0.25) (layer "B.Cu") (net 2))
 (segment (start 133.384511 82.830489) (end 140.484511 82.830489) (width 0.25) (layer "B.Cu") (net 2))
 (segment (start 133.269511 91.530489) (end 140.509511 91.530489) (width 0.25) (layer "B.Cu") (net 2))
 (segment (start 132.9 109) (end 140.515 109) (width 0.25) (layer "B.Cu") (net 2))
 (segment (start 142.6 127.5) (end 142.5 127.5) (width 0.25) (layer "B.Cu") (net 2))
 (segment (start 140.515 100.2) (end 141.9 98.815) (width 0.25) (layer "B.Cu") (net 2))
 (segment (start 133.18 127.945) (end 135.725 125.4) (width 0.25) (layer "F.Cu") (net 21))
 (segment (start 133.18 128.9) (end 133.18 127.945) (width 0.25) (layer "F.Cu") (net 21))
 (segment (start 138.265 114.065) (end 136.5 112.3) (width 0.25) (layer "F.Cu") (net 20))
 (segment (start 138.265 125.4) (end 138.265 114.065) (width 0.25) (layer "F.Cu") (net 20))
 (segment (start 136.5 112.3) (end 136.5 105.1) (width 0.25) (layer "F.Cu") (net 20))
 (via (at 136.5 105.1) (size 0.8) (drill 0.4) (layers "F.Cu" "B.Cu") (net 20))
 (segment (start 136.525 105.075) (end 139.02 105.075) (width 0.25) (layer "B.Cu") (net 20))
 (segment (start 136.5 105.1) (end 136.525 105.075) (width 0.25) (layer "B.Cu") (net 20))
 (segment (start 140.2 113.5697) (end 140.805 114.1747) (width 0.25) (layer "F.Cu") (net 29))
 (segment (start 139.02 96.275) (end 140.2 97.455) (width 0.25) (layer "F.Cu") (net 29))
 (segment (start 140.2 97.455) (end 140.2 113.5697) (width 0.25) (layer "F.Cu") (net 29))
 (segment (start 140.805 114.1747) (end 140.805 125.4) (width 0.25) (layer "F.Cu") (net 29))
 (segment (start 143.345 125.4) (end 143.345 120.955) (width 0.25) (layer "F.Cu") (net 16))
 (segment (start 145.8 118.5) (end 145.8 112.4) (width 0.25) (layer "F.Cu") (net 16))
 (segment (start 144.9 111.5) (end 144.9 105.1) (width 0.25) (layer "F.Cu") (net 16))
 (segment (start 145.8 112.4) (end 144.9 111.5) (width 0.25) (layer "F.Cu") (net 16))
 (segment (start 143.345 120.955) (end 145.8 118.5) (width 0.25) (layer "F.Cu") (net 16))
 (via (at 144.9 105.1) (size 0.8) (drill 0.4) (layers "F.Cu" "B.Cu") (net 16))
 (segment (start 144.925 105.075) (end 149.52 105.075) (width 0.25) (layer "B.Cu") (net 16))
 (segment (start 144.9 105.1) (end 144.925 105.075) (width 0.25) (layer "B.Cu") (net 16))
 (segment (start 145.885 125.4) (end 148.575489 122.709511) (width 0.25) (layer "F.Cu") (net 30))
 (segment (start 150.9 115.4) (end 150.9 96.7) (width 0.25) (layer "F.Cu") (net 30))
 (segment (start 148.575489 122.709511) (end 148.575489 117.724511) (width 0.25) (layer "F.Cu") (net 30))
 (segment (start 148.575489 117.724511) (end 150.9 115.4) (width 0.25) (layer "F.Cu") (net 30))
 (segment (start 150.9 96.7) (end 150.475 96.275) (width 0.25) (layer "F.Cu") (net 30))
 (segment (start 150.475 96.275) (end 149.52 96.275) (width 0.25) (layer "F.Cu") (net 30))
 (segment (start 149.7 112.9) (end 149.7 114.5) (width 0.25) (layer "F.Cu") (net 22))
 (segment (start 149.9 112.7) (end 149.7 112.9) (width 0.25) (layer "F.Cu") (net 22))
 (segment (start 147.7 110.5) (end 149.9 112.7) (width 0.25) (layer "F.Cu") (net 22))
 (segment (start 148 97.6) (end 148 78.6) (width 0.25) (layer "F.Cu") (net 22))
 (segment (start 147.7 97.9) (end 147.7 110.5) (width 0.25) (layer "F.Cu") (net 22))
 (segment (start 148 78.6) (end 147.1 77.7) (width 0.25) (layer "F.Cu") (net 22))
 (segment (start 147.7 97.9) (end 148 97.6) (width 0.25) (layer "F.Cu") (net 22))
 (via (at 147.1 77.7) (size 0.8) (drill 0.4) (layers "F.Cu" "B.Cu") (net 22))
 (segment (start 147.1 77.7) (end 145.6 77.7) (width 0.25) (layer "B.Cu") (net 22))
 (segment (start 144.425 78.875) (end 141.9 78.875) (width 0.25) (layer "B.Cu") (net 22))
 (segment (start 145.6 77.7) (end 144.425 78.875) (width 0.25) (layer "B.Cu") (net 22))
 (segment (start 147.4 97.5) (end 147.4 89.1) (width 0.25) (layer "F.Cu") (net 40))
 (segment (start 146.2 78.9) (end 146.3 79) (width 0.25) (layer "F.Cu") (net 40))
 (segment (start 146.935 97.965) (end 147.4 97.5) (width 0.25) (layer "F.Cu") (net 40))
 (segment (start 147.16 114.5) (end 147.16 98.19) (width 0.25) (layer "F.Cu") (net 40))
 (segment (start 147.4 89.1) (end 146.1 87.8) (width 0.25) (layer "F.Cu") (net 40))
 (segment (start 147.16 98.19) (end 146.935 97.965) (width 0.25) (layer "F.Cu") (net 40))
 (segment (start 146.1 78.9) (end 146.2 78.9) (width 0.25) (layer "F.Cu") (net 40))
 (segment (start 146.1 87.8) (end 146.1 78.9) (width 0.25) (layer "F.Cu") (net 40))
 (via (at 146.3 79) (size 0.8) (drill 0.4) (layers "F.Cu" "B.Cu") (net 40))
 (segment (start 146.3 79) (end 145.300489 79.999511) (width 0.25) (layer "B.Cu") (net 40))
 (segment (start 132.524511 79.999511) (end 131.4 78.875) (width 0.25) (layer "B.Cu") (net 40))
 (segment (start 145.300489 79.999511) (end 132.524511 79.999511) (width 0.25) (layer "B.Cu") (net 40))
 (segment (start 145.3 90.3) (end 145.3 89) (width 0.25) (layer "F.Cu") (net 34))
 (segment (start 144.1 91.5) (end 145.3 90.3) (width 0.25) (layer "F.Cu") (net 34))
 (segment (start 144.1 111.7) (end 144.1 91.5) (width 0.25) (layer "F.Cu") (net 34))
 (segment (start 144.62 114.5) (end 144.62 112.22) (width 0.25) (layer "F.Cu") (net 34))
 (segment (start 144.62 112.22) (end 144.1 111.7) (width 0.25) (layer "F.Cu") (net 34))
 (via (at 145.3 89) (size 0.8) (drill 0.4) (layers "F.Cu" "B.Cu") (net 34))
 (segment (start 139.4953 89) (end 139.1953 88.7) (width 0.25) (layer "B.Cu") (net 34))
 (segment (start 145.3 89) (end 139.4953 89) (width 0.25) (layer "B.Cu") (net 34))
 (segment (start 132.525 88.7) (end 131.4 87.575) (width 0.25) (layer "B.Cu") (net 34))
 (segment (start 139.1953 88.7) (end 132.525 88.7) (width 0.25) (layer "B.Cu") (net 34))
 (segment (start 142.08 112.72) (end 142.08 114.5) (width 0.25) (layer "F.Cu") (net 31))
 (segment (start 141.9 96.275) (end 143.3 97.675) (width 0.25) (layer "F.Cu") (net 31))
 (segment (start 143.3 97.675) (end 143.3 111.5) (width 0.25) (layer "F.Cu") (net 31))
 (segment (start 143.3 111.5) (end 142.08 112.72) (width 0.25) (layer "F.Cu") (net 31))
 (segment (start 137.5 112.46) (end 137.5 106.6) (width 0.25) (layer "F.Cu") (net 13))
 (segment (start 139.54 114.5) (end 137.5 112.46) (width 0.25) (layer "F.Cu") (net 13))
 (via (at 137.5 106.6) (size 0.8) (drill 0.4) (layers "F.Cu" "B.Cu") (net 13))
 (segment (start 140.775489 106.199511) (end 137.900489 106.199511) (width 0.25) (layer "B.Cu") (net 13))
 (segment (start 137.900489 106.199511) (end 137.5 106.6) (width 0.25) (layer "B.Cu") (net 13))
 (segment (start 141.9 105.075) (end 140.775489 106.199511) (width 0.25) (layer "B.Cu") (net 13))
 (segment (start 134.9 112.4) (end 134.9 96.3) (width 0.25) (layer "F.Cu") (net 26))
 (segment (start 137 114.5) (end 134.9 112.4) (width 0.25) (layer "F.Cu") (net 26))
 (via (at 134.9 96.3) (size 0.8) (drill 0.4) (layers "F.Cu" "B.Cu") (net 26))
 (segment (start 134.9 96.3) (end 134.875 96.275) (width 0.25) (layer "B.Cu") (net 26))
 (segment (start 134.875 96.275) (end 131.4 96.275) (width 0.25) (layer "B.Cu") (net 26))
 (segment (start 133.624511 105.775489) (end 134.1 105.3) (width 0.25) (layer "F.Cu") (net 17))
 (segment (start 133.624511 113.664511) (end 133.624511 105.775489) (width 0.25) (layer "F.Cu") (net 17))
 (segment (start 134.46 114.5) (end 133.624511 113.664511) (width 0.25) (layer "F.Cu") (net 17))
 (via (at 134.1 105.3) (size 0.8) (drill 0.4) (layers "F.Cu" "B.Cu") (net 17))
 (segment (start 133.875 105.075) (end 131.4 105.075) (width 0.25) (layer "B.Cu") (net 17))
 (segment (start 134.1 105.3) (end 133.875 105.075) (width 0.25) (layer "B.Cu") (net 17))
 (segment (start 143.4 112.9) (end 143.4 119) (width 0.25) (layer "F.Cu") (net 1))
 (segment (start 147.2 119) (end 147.16 119.04) (width 0.25) (layer "F.Cu") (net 1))
 (segment (start 140.775489 92.929211) (end 140.64952 93.05518) (width 0.25) (layer "F.Cu") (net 1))
 (segment (start 140.64952 112.44952) (end 141.1 112.9) (width 0.25) (layer "F.Cu") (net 1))
 (segment (start 140.64952 93.05518) (end 140.64952 112.44952) (width 0.25) (layer "F.Cu") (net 1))
 (segment (start 140.775489 88.724511) (end 140.775489 92.929211) (width 0.25) (layer "F.Cu") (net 1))
 (segment (start 147.16 119.04) (end 147.16 122.12) (width 0.25) (layer "F.Cu") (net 1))
 (segment (start 141.9 87.6) (end 140.775489 88.724511) (width 0.25) (layer "F.Cu") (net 1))
 (via (at 147.2 119) (size 0.8) (drill 0.4) (layers "F.Cu" "B.Cu") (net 1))
 (via (at 143.4 119) (size 0.8) (drill 0.4) (layers "F.Cu" "B.Cu") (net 1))
 (via (at 143.4 112.9) (size 0.8) (drill 0.4) (layers "F.Cu" "B.Cu") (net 1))
 (via (at 141.1 112.9) (size 0.8) (drill 0.4) (layers "F.Cu" "B.Cu") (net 1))
 (segment (start 141.1 112.9) (end 143.4 112.9) (width 0.25) (layer "B.Cu") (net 1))
 (segment (start 143.4 119) (end 147.2 119) (width 0.25) (layer "B.Cu") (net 1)))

